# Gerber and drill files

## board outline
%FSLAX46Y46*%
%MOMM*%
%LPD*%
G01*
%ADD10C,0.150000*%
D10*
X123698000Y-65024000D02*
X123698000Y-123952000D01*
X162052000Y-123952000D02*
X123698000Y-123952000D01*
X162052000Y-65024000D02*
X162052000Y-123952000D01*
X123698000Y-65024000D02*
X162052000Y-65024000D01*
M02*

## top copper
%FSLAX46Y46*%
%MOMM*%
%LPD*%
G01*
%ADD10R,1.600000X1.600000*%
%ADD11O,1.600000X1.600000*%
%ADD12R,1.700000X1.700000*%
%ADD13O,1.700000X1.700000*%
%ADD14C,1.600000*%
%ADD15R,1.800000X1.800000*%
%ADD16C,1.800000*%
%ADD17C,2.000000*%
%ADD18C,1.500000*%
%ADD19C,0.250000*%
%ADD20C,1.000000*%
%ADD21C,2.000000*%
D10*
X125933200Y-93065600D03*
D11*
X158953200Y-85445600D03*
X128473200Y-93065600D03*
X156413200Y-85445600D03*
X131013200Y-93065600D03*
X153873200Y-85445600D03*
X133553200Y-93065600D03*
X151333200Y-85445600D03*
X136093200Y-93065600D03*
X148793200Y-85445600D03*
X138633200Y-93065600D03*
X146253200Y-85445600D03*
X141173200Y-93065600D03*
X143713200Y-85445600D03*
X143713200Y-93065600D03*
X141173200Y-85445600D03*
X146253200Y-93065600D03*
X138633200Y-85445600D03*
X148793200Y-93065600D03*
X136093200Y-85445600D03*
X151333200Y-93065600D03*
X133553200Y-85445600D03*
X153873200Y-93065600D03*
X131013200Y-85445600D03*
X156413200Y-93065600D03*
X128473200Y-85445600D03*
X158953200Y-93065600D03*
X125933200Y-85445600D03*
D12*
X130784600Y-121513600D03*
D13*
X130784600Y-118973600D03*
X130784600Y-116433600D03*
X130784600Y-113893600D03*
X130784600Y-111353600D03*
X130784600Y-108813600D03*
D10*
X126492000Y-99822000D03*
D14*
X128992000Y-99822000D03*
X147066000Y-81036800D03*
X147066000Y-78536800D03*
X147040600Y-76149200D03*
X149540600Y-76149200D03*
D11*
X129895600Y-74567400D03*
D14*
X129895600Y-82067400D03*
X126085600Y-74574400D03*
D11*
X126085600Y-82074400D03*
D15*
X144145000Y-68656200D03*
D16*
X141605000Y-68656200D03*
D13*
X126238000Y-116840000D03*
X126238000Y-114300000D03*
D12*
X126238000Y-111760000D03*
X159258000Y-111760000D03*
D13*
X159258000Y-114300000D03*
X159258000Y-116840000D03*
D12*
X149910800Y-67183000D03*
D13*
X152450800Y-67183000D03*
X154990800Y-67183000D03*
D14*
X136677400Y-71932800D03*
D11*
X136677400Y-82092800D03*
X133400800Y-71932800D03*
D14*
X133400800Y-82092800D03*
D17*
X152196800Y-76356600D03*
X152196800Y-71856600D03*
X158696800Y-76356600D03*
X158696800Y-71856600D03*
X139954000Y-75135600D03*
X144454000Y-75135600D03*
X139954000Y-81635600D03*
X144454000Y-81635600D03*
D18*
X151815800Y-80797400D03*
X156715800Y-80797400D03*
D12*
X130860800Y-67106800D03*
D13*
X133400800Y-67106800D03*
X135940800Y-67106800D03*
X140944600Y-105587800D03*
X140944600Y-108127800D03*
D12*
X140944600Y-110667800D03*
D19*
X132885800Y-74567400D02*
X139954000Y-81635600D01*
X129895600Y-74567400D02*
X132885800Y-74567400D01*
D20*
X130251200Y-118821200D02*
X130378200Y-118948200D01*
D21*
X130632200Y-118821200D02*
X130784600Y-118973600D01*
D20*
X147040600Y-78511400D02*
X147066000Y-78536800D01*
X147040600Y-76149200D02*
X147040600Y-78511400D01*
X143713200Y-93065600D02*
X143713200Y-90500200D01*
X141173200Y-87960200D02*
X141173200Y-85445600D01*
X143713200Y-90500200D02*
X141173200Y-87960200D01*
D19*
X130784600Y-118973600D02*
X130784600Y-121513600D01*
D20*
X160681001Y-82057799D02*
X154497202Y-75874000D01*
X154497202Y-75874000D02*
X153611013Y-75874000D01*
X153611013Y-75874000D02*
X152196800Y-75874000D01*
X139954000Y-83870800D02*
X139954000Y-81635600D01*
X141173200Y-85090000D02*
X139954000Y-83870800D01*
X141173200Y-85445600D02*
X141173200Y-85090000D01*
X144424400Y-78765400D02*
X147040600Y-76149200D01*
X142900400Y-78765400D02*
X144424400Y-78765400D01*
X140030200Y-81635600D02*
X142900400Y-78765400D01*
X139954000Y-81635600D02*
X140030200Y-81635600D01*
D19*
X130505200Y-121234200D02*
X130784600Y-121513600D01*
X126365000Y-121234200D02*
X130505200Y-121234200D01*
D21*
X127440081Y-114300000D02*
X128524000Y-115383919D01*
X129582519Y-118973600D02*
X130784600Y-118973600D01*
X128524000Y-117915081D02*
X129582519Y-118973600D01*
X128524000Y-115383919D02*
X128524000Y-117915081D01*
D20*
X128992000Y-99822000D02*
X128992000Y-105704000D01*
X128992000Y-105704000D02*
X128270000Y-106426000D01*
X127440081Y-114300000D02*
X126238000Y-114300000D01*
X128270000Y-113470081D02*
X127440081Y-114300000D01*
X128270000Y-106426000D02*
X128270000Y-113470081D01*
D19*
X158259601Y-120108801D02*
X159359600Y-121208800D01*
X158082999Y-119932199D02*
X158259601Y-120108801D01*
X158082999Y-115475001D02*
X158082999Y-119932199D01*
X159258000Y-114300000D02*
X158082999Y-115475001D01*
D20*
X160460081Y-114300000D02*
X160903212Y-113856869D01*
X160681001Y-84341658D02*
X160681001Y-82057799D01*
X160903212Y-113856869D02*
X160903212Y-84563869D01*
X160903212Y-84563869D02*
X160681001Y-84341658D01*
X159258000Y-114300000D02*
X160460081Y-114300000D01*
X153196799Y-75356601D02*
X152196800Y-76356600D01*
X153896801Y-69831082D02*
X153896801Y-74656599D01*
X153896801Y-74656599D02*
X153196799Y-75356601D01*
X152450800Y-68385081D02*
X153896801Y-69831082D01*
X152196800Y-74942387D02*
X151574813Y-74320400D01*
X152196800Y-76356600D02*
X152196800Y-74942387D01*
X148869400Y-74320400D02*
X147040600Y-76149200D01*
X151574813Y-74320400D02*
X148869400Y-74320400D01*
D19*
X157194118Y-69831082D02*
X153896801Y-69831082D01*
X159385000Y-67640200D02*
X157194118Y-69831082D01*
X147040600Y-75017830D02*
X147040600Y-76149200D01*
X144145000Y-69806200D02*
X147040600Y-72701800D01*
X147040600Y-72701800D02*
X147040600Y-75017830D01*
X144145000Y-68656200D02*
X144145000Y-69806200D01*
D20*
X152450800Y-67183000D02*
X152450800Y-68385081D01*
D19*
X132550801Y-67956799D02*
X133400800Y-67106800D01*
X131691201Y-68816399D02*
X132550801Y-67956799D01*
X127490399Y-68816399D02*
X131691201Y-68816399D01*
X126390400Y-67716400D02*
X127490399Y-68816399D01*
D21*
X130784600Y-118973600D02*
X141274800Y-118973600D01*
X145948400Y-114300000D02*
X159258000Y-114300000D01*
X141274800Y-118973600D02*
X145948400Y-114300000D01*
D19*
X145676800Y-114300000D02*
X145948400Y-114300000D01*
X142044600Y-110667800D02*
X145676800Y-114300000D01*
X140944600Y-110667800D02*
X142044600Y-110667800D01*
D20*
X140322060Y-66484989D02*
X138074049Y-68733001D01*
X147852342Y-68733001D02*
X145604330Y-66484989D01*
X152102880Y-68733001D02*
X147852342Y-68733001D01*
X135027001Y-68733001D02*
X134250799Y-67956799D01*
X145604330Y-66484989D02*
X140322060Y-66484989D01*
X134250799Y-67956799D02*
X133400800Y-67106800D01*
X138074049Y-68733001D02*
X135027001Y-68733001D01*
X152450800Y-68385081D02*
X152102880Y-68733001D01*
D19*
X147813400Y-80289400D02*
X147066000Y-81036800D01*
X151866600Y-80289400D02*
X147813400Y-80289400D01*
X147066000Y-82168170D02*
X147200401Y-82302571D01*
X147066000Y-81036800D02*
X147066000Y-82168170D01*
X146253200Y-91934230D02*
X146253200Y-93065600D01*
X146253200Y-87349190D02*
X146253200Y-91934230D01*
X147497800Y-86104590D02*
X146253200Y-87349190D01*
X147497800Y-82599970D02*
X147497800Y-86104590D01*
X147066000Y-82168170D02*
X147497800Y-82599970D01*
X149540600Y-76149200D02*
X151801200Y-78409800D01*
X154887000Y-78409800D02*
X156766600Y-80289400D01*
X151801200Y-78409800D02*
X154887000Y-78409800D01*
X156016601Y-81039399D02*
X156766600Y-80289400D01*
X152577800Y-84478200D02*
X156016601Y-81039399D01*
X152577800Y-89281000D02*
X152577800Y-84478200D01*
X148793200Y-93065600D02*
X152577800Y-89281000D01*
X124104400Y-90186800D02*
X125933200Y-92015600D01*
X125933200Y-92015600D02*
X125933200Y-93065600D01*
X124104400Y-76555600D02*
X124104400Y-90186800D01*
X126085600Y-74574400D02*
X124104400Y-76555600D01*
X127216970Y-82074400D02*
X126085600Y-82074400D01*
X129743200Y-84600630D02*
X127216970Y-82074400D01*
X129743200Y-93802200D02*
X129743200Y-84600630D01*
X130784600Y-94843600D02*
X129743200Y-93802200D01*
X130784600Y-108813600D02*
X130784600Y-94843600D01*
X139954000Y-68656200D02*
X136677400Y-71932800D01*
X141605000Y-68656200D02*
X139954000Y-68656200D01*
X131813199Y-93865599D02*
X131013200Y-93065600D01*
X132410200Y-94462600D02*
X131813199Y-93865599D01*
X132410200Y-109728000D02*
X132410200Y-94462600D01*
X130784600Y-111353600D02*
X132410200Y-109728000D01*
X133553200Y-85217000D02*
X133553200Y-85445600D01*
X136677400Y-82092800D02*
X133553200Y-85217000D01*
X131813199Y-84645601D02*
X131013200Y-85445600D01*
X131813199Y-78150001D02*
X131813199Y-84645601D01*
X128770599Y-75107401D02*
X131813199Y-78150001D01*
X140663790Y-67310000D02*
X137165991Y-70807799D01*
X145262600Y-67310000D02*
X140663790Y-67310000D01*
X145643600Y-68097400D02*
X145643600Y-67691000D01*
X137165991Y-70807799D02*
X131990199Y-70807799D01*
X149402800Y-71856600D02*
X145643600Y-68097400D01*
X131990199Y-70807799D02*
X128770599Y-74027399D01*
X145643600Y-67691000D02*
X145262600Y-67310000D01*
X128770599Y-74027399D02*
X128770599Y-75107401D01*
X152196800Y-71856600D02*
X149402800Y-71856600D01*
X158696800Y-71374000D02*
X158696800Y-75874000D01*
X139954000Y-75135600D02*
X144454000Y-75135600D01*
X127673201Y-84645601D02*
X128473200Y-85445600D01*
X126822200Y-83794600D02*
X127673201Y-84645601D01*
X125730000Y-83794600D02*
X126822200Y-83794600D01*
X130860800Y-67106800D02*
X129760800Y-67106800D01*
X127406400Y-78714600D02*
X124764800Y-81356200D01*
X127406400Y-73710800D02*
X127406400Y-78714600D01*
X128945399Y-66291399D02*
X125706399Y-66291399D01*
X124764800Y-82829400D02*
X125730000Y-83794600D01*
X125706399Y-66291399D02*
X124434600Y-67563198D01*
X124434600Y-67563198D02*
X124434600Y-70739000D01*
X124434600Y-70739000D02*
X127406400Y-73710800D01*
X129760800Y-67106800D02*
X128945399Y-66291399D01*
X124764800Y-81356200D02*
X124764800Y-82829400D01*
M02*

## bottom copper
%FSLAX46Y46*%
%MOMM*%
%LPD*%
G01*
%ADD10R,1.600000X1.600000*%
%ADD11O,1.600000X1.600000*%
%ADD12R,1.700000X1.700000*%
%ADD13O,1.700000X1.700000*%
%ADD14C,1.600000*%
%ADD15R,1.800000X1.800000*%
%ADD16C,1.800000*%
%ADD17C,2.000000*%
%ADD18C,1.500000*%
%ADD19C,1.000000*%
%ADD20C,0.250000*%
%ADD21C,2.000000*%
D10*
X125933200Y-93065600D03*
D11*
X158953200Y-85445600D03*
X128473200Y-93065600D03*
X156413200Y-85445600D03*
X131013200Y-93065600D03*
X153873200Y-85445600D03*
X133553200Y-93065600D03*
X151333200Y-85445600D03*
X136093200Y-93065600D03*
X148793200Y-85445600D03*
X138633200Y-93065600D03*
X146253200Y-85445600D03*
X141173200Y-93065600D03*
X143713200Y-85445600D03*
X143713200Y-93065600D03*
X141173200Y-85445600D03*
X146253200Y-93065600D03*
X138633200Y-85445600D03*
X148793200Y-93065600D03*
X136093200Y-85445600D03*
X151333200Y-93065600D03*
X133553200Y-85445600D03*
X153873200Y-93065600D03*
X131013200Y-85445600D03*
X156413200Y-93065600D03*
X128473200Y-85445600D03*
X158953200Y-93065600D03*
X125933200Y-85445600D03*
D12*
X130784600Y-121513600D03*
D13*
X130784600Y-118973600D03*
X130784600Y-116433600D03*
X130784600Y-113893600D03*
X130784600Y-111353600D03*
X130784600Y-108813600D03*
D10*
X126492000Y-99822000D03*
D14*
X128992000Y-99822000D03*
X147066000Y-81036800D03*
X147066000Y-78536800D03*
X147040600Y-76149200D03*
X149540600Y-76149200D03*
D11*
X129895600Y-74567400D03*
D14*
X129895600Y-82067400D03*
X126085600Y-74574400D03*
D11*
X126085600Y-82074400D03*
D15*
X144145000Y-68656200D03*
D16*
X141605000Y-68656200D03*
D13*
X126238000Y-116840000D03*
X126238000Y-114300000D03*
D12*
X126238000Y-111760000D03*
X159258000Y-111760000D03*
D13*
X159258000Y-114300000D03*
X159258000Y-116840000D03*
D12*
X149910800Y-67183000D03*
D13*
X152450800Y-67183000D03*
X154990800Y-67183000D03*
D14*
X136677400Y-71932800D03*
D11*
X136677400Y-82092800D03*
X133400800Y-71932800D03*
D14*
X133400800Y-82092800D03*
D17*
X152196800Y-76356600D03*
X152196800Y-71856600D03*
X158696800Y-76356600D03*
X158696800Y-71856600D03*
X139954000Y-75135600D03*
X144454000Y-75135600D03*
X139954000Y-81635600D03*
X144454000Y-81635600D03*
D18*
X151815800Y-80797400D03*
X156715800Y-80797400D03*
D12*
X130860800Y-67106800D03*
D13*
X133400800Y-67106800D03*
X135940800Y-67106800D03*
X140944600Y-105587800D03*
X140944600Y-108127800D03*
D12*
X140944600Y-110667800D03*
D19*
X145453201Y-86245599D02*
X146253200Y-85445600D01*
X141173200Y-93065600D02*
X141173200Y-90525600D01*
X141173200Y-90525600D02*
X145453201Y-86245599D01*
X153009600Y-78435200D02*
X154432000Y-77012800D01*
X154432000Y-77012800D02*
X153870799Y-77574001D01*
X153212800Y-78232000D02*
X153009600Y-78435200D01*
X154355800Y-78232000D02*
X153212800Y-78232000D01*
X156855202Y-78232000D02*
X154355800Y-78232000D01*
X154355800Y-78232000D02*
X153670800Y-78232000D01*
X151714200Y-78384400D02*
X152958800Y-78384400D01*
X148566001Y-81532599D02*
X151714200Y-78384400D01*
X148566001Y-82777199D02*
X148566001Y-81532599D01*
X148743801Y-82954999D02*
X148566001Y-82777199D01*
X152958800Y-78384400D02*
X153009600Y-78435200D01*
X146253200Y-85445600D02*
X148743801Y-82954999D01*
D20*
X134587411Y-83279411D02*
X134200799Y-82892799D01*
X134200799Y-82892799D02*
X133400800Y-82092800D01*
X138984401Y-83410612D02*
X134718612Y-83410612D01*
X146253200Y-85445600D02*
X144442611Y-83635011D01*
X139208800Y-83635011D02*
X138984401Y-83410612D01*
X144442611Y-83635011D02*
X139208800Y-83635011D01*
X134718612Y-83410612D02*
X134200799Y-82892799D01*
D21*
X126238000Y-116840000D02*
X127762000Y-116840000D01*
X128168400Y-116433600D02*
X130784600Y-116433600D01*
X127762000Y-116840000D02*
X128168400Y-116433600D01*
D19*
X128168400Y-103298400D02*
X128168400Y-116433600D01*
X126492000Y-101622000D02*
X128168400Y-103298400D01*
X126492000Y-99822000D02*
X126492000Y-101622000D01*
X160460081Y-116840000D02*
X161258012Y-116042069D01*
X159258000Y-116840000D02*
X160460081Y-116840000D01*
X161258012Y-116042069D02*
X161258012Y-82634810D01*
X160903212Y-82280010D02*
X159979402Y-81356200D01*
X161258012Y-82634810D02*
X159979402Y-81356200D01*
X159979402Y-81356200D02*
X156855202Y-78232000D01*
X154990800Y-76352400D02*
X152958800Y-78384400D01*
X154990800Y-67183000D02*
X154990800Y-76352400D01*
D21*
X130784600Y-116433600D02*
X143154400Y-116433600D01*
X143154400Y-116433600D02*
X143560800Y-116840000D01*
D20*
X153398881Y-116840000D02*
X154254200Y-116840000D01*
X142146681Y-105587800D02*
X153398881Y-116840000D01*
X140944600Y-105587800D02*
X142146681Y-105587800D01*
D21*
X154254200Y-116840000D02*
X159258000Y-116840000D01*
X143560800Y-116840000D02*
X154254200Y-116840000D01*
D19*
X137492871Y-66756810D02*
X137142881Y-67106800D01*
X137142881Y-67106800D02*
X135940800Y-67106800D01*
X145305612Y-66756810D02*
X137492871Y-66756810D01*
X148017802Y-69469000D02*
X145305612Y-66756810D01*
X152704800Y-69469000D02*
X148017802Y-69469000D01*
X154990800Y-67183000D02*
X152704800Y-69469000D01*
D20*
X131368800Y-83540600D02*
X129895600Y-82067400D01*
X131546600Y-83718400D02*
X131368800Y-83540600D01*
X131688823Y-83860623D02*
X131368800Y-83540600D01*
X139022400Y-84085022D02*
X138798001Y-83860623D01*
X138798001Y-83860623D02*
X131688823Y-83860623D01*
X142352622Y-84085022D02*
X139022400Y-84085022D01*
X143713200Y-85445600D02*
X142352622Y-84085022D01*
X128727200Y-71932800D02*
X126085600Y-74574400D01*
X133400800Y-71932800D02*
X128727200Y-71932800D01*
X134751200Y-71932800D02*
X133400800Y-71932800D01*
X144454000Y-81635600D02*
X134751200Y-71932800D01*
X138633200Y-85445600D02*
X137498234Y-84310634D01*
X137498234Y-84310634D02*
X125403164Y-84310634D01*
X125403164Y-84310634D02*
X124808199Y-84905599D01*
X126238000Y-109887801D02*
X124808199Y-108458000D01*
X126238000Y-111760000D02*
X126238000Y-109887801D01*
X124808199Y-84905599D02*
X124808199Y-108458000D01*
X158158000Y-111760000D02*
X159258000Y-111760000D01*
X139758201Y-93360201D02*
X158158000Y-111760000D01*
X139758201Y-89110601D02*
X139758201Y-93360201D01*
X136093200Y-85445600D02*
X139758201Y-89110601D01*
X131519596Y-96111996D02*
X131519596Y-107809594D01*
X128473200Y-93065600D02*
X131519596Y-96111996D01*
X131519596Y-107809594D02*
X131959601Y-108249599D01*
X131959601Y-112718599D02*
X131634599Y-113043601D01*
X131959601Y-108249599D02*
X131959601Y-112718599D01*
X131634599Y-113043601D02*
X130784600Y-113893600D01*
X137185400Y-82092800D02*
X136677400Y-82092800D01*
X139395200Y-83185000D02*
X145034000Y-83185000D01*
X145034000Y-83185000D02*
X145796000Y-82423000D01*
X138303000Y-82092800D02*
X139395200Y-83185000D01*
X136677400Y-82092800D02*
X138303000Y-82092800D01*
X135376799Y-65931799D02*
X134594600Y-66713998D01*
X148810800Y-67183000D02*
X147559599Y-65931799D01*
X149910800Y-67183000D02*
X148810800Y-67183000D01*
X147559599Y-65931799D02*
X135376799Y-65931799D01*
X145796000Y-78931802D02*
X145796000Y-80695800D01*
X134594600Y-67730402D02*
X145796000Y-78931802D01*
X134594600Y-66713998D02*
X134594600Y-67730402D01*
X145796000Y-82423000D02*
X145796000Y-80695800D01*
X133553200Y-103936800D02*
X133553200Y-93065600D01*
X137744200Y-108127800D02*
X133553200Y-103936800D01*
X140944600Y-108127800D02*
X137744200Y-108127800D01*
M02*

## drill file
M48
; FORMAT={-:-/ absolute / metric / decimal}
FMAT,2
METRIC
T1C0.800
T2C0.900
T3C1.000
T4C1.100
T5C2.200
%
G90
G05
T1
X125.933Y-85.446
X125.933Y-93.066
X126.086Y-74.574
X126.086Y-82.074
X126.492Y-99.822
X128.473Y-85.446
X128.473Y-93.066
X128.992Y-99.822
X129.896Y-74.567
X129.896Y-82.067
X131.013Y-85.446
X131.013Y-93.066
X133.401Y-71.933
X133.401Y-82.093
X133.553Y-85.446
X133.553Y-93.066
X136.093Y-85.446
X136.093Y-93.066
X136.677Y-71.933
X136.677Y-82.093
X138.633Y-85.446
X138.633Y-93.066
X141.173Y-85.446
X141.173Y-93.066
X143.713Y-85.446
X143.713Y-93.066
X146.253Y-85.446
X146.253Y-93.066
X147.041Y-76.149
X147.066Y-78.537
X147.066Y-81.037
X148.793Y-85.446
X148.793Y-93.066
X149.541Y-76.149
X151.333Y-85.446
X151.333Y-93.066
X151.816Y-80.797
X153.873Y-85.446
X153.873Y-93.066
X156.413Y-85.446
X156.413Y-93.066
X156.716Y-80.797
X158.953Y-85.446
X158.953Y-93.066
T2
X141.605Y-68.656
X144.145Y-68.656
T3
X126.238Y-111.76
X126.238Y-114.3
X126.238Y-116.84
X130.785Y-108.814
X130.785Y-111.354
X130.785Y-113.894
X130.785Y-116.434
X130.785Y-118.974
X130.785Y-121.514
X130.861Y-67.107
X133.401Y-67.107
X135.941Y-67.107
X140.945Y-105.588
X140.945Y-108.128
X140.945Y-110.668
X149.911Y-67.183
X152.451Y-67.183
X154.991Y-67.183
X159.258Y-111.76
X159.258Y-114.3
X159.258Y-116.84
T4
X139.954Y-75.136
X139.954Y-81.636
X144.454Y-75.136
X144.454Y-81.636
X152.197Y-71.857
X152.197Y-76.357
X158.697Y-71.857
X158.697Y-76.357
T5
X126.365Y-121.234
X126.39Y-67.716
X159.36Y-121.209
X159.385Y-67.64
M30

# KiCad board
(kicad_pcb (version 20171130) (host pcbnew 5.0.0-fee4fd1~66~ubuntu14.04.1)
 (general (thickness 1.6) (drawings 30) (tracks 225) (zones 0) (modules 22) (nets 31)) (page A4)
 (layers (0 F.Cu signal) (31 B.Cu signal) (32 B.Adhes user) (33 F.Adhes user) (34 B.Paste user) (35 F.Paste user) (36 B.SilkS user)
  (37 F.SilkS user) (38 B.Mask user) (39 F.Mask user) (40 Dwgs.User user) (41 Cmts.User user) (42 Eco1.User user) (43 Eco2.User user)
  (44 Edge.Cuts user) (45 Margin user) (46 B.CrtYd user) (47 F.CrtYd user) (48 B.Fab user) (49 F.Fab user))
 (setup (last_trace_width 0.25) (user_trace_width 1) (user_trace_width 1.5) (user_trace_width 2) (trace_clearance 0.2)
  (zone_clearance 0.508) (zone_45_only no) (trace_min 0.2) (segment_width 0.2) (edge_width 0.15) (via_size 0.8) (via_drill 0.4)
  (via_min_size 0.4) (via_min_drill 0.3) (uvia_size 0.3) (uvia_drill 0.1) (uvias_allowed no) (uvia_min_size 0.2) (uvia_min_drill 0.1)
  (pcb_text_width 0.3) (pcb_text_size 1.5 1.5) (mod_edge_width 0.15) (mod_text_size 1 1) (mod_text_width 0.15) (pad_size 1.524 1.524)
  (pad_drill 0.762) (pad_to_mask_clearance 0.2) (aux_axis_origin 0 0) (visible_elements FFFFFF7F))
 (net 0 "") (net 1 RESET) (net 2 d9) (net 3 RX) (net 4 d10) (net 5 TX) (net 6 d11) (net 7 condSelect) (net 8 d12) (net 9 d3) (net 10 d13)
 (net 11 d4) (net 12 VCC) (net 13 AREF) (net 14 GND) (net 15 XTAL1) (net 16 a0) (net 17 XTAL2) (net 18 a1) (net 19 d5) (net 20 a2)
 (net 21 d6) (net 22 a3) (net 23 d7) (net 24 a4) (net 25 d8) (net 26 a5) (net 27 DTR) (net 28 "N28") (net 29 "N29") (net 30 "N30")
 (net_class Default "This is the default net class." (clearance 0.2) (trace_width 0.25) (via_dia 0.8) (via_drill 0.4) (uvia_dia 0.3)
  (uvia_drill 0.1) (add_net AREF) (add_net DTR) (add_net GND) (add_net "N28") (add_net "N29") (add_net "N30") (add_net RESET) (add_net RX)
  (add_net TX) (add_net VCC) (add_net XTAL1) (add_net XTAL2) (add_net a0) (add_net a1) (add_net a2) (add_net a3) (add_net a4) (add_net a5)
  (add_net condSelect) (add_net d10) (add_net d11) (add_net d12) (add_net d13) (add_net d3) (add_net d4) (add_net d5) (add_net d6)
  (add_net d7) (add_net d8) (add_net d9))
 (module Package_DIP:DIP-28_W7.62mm (layer F.Cu) (at 125.9332 93.0656 90)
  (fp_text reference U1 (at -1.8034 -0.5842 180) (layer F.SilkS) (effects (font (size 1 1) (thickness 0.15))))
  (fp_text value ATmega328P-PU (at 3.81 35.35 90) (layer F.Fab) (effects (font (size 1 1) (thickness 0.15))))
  (pad 1 thru_hole rect (at 0 0 90) (size 1.6 1.6) (drill 0.8) (layers *.Cu *.Mask) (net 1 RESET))
  (pad 15 thru_hole oval (at 7.62 33.02 90) (size 1.6 1.6) (drill 0.8) (layers *.Cu *.Mask) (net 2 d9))
  (pad 2 thru_hole oval (at 0 2.54 90) (size 1.6 1.6) (drill 0.8) (layers *.Cu *.Mask) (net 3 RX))
  (pad 16 thru_hole oval (at 7.62 30.48 90) (size 1.6 1.6) (drill 0.8) (layers *.Cu *.Mask) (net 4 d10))
  (pad 3 thru_hole oval (at 0 5.08 90) (size 1.6 1.6) (drill 0.8) (layers *.Cu *.Mask) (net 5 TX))
  (pad 17 thru_hole oval (at 7.62 27.94 90) (size 1.6 1.6) (drill 0.8) (layers *.Cu *.Mask) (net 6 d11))
  (pad 4 thru_hole oval (at 0 7.62 90) (size 1.6 1.6) (drill 0.8) (layers *.Cu *.Mask) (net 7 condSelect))
  (pad 18 thru_hole oval (at 7.62 25.4 90) (size 1.6 1.6) (drill 0.8) (layers *.Cu *.Mask) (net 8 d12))
  (pad 5 thru_hole oval (at 0 10.16 90) (size 1.6 1.6) (drill 0.8) (layers *.Cu *.Mask) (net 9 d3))
  (pad 19 thru_hole oval (at 7.62 22.86 90) (size 1.6 1.6) (drill 0.8) (layers *.Cu *.Mask) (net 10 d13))
  (pad 6 thru_hole oval (at 0 12.7 90) (size 1.6 1.6) (drill 0.8) (layers *.Cu *.Mask) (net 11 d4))
  (pad 20 thru_hole oval (at 7.62 20.32 90) (size 1.6 1.6) (drill 0.8) (layers *.Cu *.Mask) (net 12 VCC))
  (pad 7 thru_hole oval (at 0 15.24 90) (size 1.6 1.6) (drill 0.8) (layers *.Cu *.Mask) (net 12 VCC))
  (pad 21 thru_hole oval (at 7.62 17.78 90) (size 1.6 1.6) (drill 0.8) (layers *.Cu *.Mask) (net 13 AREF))
  (pad 8 thru_hole oval (at 0 17.78 90) (size 1.6 1.6) (drill 0.8) (layers *.Cu *.Mask) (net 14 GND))
  (pad 22 thru_hole oval (at 7.62 15.24 90) (size 1.6 1.6) (drill 0.8) (layers *.Cu *.Mask) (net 14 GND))
  (pad 9 thru_hole oval (at 0 20.32 90) (size 1.6 1.6) (drill 0.8) (layers *.Cu *.Mask) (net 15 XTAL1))
  (pad 23 thru_hole oval (at 7.62 12.7 90) (size 1.6 1.6) (drill 0.8) (layers *.Cu *.Mask) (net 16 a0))
  (pad 10 thru_hole oval (at 0 22.86 90) (size 1.6 1.6) (drill 0.8) (layers *.Cu *.Mask) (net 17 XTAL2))
  (pad 24 thru_hole oval (at 7.62 10.16 90) (size 1.6 1.6) (drill 0.8) (layers *.Cu *.Mask) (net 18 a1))
  (pad 11 thru_hole oval (at 0 25.4 90) (size 1.6 1.6) (drill 0.8) (layers *.Cu *.Mask) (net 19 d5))
  (pad 25 thru_hole oval (at 7.62 7.62 90) (size 1.6 1.6) (drill 0.8) (layers *.Cu *.Mask) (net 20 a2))
  (pad 12 thru_hole oval (at 0 27.94 90) (size 1.6 1.6) (drill 0.8) (layers *.Cu *.Mask) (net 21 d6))
  (pad 26 thru_hole oval (at 7.62 5.08 90) (size 1.6 1.6) (drill 0.8) (layers *.Cu *.Mask) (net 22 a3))
  (pad 13 thru_hole oval (at 0 30.48 90) (size 1.6 1.6) (drill 0.8) (layers *.Cu *.Mask) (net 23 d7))
  (pad 27 thru_hole oval (at 7.62 2.54 90) (size 1.6 1.6) (drill 0.8) (layers *.Cu *.Mask) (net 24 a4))
  (pad 14 thru_hole oval (at 0 33.02 90) (size 1.6 1.6) (drill 0.8) (layers *.Cu *.Mask) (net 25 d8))
  (pad 28 thru_hole oval (at 7.62 0 90) (size 1.6 1.6) (drill 0.8) (layers *.Cu *.Mask) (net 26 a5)))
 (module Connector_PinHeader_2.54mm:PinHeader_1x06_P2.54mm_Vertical (layer F.Cu) (at 130.7846 121.5136 180)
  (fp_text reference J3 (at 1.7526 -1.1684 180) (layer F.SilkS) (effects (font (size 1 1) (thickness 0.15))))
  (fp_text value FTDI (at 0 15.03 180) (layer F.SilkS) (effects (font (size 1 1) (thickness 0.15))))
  (pad 1 thru_hole rect (at 0 0 180) (size 1.7 1.7) (drill 1) (layers *.Cu *.Mask) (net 14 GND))
  (pad 2 thru_hole oval (at 0 2.54 180) (size 1.7 1.7) (drill 1) (layers *.Cu *.Mask) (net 14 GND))
  (pad 3 thru_hole oval (at 0 5.08 180) (size 1.7 1.7) (drill 1) (layers *.Cu *.Mask) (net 12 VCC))
  (pad 4 thru_hole oval (at 0 7.62 180) (size 1.7 1.7) (drill 1) (layers *.Cu *.Mask) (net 3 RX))
  (pad 5 thru_hole oval (at 0 10.16 180) (size 1.7 1.7) (drill 1) (layers *.Cu *.Mask) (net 5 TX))
  (pad 6 thru_hole oval (at 0 12.7 180) (size 1.7 1.7) (drill 1) (layers *.Cu *.Mask) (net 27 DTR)))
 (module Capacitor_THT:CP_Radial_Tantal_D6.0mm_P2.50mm (layer F.Cu) (at 126.492 99.822)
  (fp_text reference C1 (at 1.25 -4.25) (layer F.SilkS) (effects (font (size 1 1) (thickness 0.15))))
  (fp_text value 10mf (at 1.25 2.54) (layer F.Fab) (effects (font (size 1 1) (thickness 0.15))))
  (pad 1 thru_hole rect (at 0 0) (size 1.6 1.6) (drill 0.8) (layers *.Cu *.Mask) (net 12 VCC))
  (pad 2 thru_hole circle (at 2.5 0) (size 1.6 1.6) (drill 0.8) (layers *.Cu *.Mask) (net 14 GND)))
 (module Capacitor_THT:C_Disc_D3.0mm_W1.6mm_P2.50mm (layer F.Cu) (at 147.066 78.5368 270)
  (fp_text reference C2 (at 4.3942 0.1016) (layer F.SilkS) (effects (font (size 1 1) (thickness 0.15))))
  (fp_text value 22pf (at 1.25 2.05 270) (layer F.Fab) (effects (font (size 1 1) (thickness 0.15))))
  (pad 2 thru_hole circle (at 2.5 0 270) (size 1.6 1.6) (drill 0.8) (layers *.Cu *.Mask) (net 15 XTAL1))
  (pad 1 thru_hole circle (at 0 0 270) (size 1.6 1.6) (drill 0.8) (layers *.Cu *.Mask) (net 14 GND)))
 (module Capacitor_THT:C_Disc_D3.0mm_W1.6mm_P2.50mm (layer F.Cu) (at 147.0406 76.1492)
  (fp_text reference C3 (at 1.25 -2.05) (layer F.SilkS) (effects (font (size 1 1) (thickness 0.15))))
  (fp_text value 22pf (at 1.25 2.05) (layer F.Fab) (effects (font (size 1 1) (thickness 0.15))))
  (pad 1 thru_hole circle (at 0 0) (size 1.6 1.6) (drill 0.8) (layers *.Cu *.Mask) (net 14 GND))
  (pad 2 thru_hole circle (at 2.5 0) (size 1.6 1.6) (drill 0.8) (layers *.Cu *.Mask) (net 17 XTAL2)))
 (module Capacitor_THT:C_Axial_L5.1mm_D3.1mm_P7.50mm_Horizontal (layer F.Cu) (at 129.8956 82.0674 90)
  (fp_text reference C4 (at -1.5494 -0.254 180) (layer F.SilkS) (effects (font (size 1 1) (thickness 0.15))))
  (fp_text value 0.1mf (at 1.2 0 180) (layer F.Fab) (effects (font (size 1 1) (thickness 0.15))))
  (pad 2 thru_hole oval (at 7.5 0 90) (size 1.6 1.6) (drill 0.8) (layers *.Cu *.Mask) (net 14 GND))
  (pad 1 thru_hole circle (at 0 0 90) (size 1.6 1.6) (drill 0.8) (layers *.Cu *.Mask) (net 13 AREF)))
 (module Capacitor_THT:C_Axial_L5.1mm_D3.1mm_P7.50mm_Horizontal (layer F.Cu) (at 126.0856 74.5744 270)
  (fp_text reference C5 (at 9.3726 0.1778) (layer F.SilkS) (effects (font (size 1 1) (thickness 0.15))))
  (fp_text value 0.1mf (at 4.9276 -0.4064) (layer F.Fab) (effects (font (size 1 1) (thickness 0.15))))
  (pad 1 thru_hole circle (at 0 0 270) (size 1.6 1.6) (drill 0.8) (layers *.Cu *.Mask) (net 1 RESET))
  (pad 2 thru_hole oval (at 7.5 0 270) (size 1.6 1.6) (drill 0.8) (layers *.Cu *.Mask) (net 27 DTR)))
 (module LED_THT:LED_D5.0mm (layer F.Cu) (at 144.145 68.6562 180)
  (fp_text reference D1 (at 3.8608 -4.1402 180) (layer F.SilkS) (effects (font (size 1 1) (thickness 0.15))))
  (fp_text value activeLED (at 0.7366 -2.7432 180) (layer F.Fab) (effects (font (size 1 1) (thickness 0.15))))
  (pad 1 thru_hole rect (at 0 0 180) (size 1.8 1.8) (drill 0.9) (layers *.Cu *.Mask) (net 14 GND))
  (pad 2 thru_hole circle (at 2.54 0 180) (size 1.8 1.8) (drill 0.9) (layers *.Cu *.Mask) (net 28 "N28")))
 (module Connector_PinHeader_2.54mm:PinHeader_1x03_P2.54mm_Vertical (layer F.Cu) (at 126.238 111.76)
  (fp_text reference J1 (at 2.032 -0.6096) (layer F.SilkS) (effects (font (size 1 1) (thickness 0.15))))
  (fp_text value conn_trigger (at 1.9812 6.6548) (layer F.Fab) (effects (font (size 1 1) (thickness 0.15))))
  (pad 3 thru_hole oval (at 0 5.08) (size 1.7 1.7) (drill 1) (layers *.Cu *.Mask) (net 12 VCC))
  (pad 2 thru_hole oval (at 0 2.54) (size 1.7 1.7) (drill 1) (layers *.Cu *.Mask) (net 14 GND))
  (pad 1 thru_hole rect (at 0 0) (size 1.7 1.7) (drill 1) (layers *.Cu *.Mask) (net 16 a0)))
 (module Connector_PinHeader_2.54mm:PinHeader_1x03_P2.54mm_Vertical (layer F.Cu) (at 159.258 111.76)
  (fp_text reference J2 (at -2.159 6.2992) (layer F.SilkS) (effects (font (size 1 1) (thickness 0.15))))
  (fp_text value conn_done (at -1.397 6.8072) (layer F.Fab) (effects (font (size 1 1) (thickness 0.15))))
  (pad 1 thru_hole rect (at 0 0) (size 1.7 1.7) (drill 1) (layers *.Cu *.Mask) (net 18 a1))
  (pad 2 thru_hole oval (at 0 2.54) (size 1.7 1.7) (drill 1) (layers *.Cu *.Mask) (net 14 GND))
  (pad 3 thru_hole oval (at 0 5.08) (size 1.7 1.7) (drill 1) (layers *.Cu *.Mask) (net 12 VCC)))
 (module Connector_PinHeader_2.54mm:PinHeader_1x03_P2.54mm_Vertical (layer F.Cu) (at 149.9108 67.183 90)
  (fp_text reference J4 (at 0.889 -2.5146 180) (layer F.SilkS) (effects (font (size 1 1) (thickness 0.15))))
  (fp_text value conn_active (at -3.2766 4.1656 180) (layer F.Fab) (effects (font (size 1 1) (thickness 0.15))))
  (pad 1 thru_hole rect (at 0 0 90) (size 1.7 1.7) (drill 1) (layers *.Cu *.Mask) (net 20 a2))
  (pad 2 thru_hole oval (at 0 2.54 90) (size 1.7 1.7) (drill 1) (layers *.Cu *.Mask) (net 14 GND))
  (pad 3 thru_hole oval (at 0 5.08 90) (size 1.7 1.7) (drill 1) (layers *.Cu *.Mask) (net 12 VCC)))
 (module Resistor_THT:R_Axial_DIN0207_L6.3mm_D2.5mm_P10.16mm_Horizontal (layer F.Cu) (at 136.6774 71.9328 270)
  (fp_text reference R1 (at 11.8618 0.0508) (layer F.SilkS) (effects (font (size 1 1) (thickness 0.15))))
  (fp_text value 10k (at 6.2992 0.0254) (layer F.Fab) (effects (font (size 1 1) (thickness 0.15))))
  (pad 1 thru_hole circle (at 0 0 270) (size 1.6 1.6) (drill 0.8) (layers *.Cu *.Mask) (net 28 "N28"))
  (pad 2 thru_hole oval (at 10.16 0 270) (size 1.6 1.6) (drill 0.8) (layers *.Cu *.Mask) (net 20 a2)))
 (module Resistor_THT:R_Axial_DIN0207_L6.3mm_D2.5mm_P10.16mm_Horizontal (layer F.Cu) (at 133.4008 82.0928 90)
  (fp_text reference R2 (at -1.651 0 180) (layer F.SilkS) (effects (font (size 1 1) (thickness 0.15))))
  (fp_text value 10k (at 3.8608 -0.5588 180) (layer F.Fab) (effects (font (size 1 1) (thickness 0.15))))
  (pad 2 thru_hole oval (at 10.16 0 90) (size 1.6 1.6) (drill 0.8) (layers *.Cu *.Mask) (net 1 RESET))
  (pad 1 thru_hole circle (at 0 0 90) (size 1.6 1.6) (drill 0.8) (layers *.Cu *.Mask) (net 12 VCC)))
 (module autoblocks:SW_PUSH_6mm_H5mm (layer F.Cu) (at 152.1968 71.8566)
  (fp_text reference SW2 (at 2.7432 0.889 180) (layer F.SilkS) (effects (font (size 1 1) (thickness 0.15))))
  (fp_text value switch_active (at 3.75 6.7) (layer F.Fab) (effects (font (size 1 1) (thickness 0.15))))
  (pad 2 thru_hole circle (at 0 4.5 90) (size 2 2) (drill 1.1) (layers *.Cu *.Mask) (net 14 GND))
  (pad 1 thru_hole circle (at 0 0 90) (size 2 2) (drill 1.1) (layers *.Cu *.Mask) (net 22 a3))
  (pad 4 thru_hole circle (at 6.5 4.5 90) (size 2 2) (drill 1.1) (layers *.Cu *.Mask) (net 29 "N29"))
  (pad 3 thru_hole circle (at 6.5 0 90) (size 2 2) (drill 1.1) (layers *.Cu *.Mask) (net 29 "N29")))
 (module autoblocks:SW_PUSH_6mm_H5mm (layer F.Cu) (at 139.954 81.6356 90)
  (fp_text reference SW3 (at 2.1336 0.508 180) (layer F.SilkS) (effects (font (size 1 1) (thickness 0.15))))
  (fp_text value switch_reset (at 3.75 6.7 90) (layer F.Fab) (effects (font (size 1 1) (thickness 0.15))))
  (pad 3 thru_hole circle (at 6.5 0 180) (size 2 2) (drill 1.1) (layers *.Cu *.Mask) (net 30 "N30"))
  (pad 4 thru_hole circle (at 6.5 4.5 180) (size 2 2) (drill 1.1) (layers *.Cu *.Mask) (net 30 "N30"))
  (pad 1 thru_hole circle (at 0 0 180) (size 2 2) (drill 1.1) (layers *.Cu *.Mask) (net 14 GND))
  (pad 2 thru_hole circle (at 0 4.5 180) (size 2 2) (drill 1.1) (layers *.Cu *.Mask) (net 1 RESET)))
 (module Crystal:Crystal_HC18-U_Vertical (layer F.Cu) (at 151.8158 80.7974)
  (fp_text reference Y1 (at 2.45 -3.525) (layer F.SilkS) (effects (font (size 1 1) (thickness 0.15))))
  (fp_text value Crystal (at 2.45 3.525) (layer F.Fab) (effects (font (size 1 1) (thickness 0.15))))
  (pad 1 thru_hole circle (at 0 0) (size 1.5 1.5) (drill 0.8) (layers *.Cu *.Mask) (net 15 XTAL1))
  (pad 2 thru_hole circle (at 4.9 0) (size 1.5 1.5) (drill 0.8) (layers *.Cu *.Mask) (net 17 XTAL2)))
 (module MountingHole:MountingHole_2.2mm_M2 (layer F.Cu) (at 126.365 121.2342)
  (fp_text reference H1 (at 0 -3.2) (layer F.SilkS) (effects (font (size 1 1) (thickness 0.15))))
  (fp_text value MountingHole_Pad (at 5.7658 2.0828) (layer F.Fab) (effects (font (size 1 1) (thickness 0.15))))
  (pad 1 np_thru_hole circle (at 0 0) (size 2.2 2.2) (drill 2.2) (layers *.Cu *.Mask) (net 14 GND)))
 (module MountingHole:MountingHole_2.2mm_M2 (layer F.Cu) (at 159.3596 121.2088)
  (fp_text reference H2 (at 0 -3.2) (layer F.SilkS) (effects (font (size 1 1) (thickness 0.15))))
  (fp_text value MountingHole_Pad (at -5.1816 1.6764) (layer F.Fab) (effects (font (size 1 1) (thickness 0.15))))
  (pad 1 np_thru_hole circle (at 0 0) (size 2.2 2.2) (drill 2.2) (layers *.Cu *.Mask) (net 14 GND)))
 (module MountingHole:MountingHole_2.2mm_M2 (layer F.Cu) (at 159.385 67.6402)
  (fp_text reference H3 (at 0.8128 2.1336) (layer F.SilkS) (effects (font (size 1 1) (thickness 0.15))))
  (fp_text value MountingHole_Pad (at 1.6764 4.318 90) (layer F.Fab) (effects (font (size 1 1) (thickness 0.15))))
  (pad 1 np_thru_hole circle (at 0 0) (size 2.2 2.2) (drill 2.2) (layers *.Cu *.Mask) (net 14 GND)))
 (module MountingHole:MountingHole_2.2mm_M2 (layer F.Cu) (at 126.3904 67.7164)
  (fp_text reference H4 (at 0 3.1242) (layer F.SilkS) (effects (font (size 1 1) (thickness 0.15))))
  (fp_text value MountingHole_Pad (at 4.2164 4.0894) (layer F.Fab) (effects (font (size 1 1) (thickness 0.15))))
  (pad 1 np_thru_hole circle (at 0 0) (size 2.2 2.2) (drill 2.2) (layers *.Cu *.Mask) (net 14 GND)))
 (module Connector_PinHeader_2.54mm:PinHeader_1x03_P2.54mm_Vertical (layer F.Cu) (at 130.8608 67.1068 90)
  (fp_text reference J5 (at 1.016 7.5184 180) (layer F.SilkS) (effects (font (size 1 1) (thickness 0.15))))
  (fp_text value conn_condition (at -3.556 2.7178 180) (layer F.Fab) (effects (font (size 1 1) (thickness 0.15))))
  (pad 1 thru_hole rect (at 0 0 90) (size 1.7 1.7) (drill 1) (layers *.Cu *.Mask) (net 24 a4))
  (pad 2 thru_hole oval (at 0 2.54 90) (size 1.7 1.7) (drill 1) (layers *.Cu *.Mask) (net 14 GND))
  (pad 3 thru_hole oval (at 0 5.08 90) (size 1.7 1.7) (drill 1) (layers *.Cu *.Mask) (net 12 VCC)))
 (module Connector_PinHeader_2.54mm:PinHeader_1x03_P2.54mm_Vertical (layer F.Cu) (at 140.9446 110.6678 180)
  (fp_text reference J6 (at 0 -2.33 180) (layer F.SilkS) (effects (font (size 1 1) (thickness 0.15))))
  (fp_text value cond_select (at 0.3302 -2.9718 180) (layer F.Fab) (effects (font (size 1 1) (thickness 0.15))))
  (pad 3 thru_hole oval (at 0 5.08 180) (size 1.7 1.7) (drill 1) (layers *.Cu *.Mask) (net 12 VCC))
  (pad 2 thru_hole oval (at 0 2.54 180) (size 1.7 1.7) (drill 1) (layers *.Cu *.Mask) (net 7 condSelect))
  (pad 1 thru_hole rect (at 0 0 180) (size 1.7 1.7) (drill 1) (layers *.Cu *.Mask) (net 14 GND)))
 (gr_line (start 123.698 65.024) (end 123.698 123.952) (layer Edge.Cuts) (width 0.15))
 (gr_line (start 162.052 123.952) (end 123.698 123.952) (layer Edge.Cuts) (width 0.15))
 (gr_line (start 162.052 65.024) (end 162.052 123.952) (layer Edge.Cuts) (width 0.15))
 (gr_line (start 123.698 65.024) (end 162.052 65.024) (layer Edge.Cuts) (width 0.15))
 (segment (start 132.8858 74.5674) (end 139.954 81.6356) (width 0.25) (layer F.Cu) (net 14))
 (segment (start 129.8956 74.5674) (end 132.8858 74.5674) (width 0.25) (layer F.Cu) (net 14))
 (segment (start 130.2512 118.8212) (end 130.3782 118.9482) (width 1) (layer F.Cu) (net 14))
 (segment (start 130.6322 118.8212) (end 130.7846 118.9736) (width 2) (layer F.Cu) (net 14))
 (segment (start 147.0406 78.5114) (end 147.066 78.5368) (width 1) (layer F.Cu) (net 14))
 (segment (start 147.0406 76.1492) (end 147.0406 78.5114) (width 1) (layer F.Cu) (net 14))
 (segment (start 143.7132 93.0656) (end 143.7132 90.5002) (width 1) (layer F.Cu) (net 14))
 (segment (start 141.1732 87.9602) (end 141.1732 85.4456) (width 1) (layer F.Cu) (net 14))
 (segment (start 143.7132 90.5002) (end 141.1732 87.9602) (width 1) (layer F.Cu) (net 14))
 (segment (start 130.7846 118.9736) (end 130.7846 121.5136) (width 0.25) (layer F.Cu) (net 14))
 (segment (start 160.681001 82.057799) (end 154.497202 75.874) (width 1) (layer F.Cu) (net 14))
 (segment (start 154.497202 75.874) (end 153.611013 75.874) (width 1) (layer F.Cu) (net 14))
 (segment (start 153.611013 75.874) (end 152.1968 75.874) (width 1) (layer F.Cu) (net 14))
 (segment (start 139.954 83.8708) (end 139.954 81.6356) (width 1) (layer F.Cu) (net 14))
 (segment (start 141.1732 85.09) (end 139.954 83.8708) (width 1) (layer F.Cu) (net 14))
 (segment (start 141.1732 85.4456) (end 141.1732 85.09) (width 1) (layer F.Cu) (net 14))
 (segment (start 144.4244 78.7654) (end 147.0406 76.1492) (width 1) (layer F.Cu) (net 14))
 (segment (start 142.9004 78.7654) (end 144.4244 78.7654) (width 1) (layer F.Cu) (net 14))
 (segment (start 140.0302 81.6356) (end 142.9004 78.7654) (width 1) (layer F.Cu) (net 14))
 (segment (start 139.954 81.6356) (end 140.0302 81.6356) (width 1) (layer F.Cu) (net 14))
 (segment (start 130.5052 121.2342) (end 130.7846 121.5136) (width 0.25) (layer F.Cu) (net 14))
 (segment (start 126.365 121.2342) (end 130.5052 121.2342) (width 0.25) (layer F.Cu) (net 14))
 (segment (start 127.440081 114.3) (end 128.524 115.383919) (width 2) (layer F.Cu) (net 14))
 (segment (start 129.582519 118.9736) (end 130.7846 118.9736) (width 2) (layer F.Cu) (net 14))
 (segment (start 128.524 117.915081) (end 129.582519 118.9736) (width 2) (layer F.Cu) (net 14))
 (segment (start 128.524 115.383919) (end 128.524 117.915081) (width 2) (layer F.Cu) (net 14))
 (segment (start 128.992 99.822) (end 128.992 105.704) (width 1) (layer F.Cu) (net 14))
 (segment (start 128.992 105.704) (end 128.27 106.426) (width 1) (layer F.Cu) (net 14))
 (segment (start 127.440081 114.3) (end 126.238 114.3) (width 1) (layer F.Cu) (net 14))
 (segment (start 128.27 113.470081) (end 127.440081 114.3) (width 1) (layer F.Cu) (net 14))
 (segment (start 128.27 106.426) (end 128.27 113.470081) (width 1) (layer F.Cu) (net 14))
 (segment (start 158.259601 120.108801) (end 159.3596 121.2088) (width 0.25) (layer F.Cu) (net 14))
 (segment (start 158.082999 119.932199) (end 158.259601 120.108801) (width 0.25) (layer F.Cu) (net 14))
 (segment (start 158.082999 115.475001) (end 158.082999 119.932199) (width 0.25) (layer F.Cu) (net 14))
 (segment (start 159.258 114.3) (end 158.082999 115.475001) (width 0.25) (layer F.Cu) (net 14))
 (segment (start 160.460081 114.3) (end 160.903212 113.856869) (width 1) (layer F.Cu) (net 14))
 (segment (start 160.681001 84.341658) (end 160.681001 82.057799) (width 1) (layer F.Cu) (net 14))
 (segment (start 160.903212 113.856869) (end 160.903212 84.563869) (width 1) (layer F.Cu) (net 14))
 (segment (start 160.903212 84.563869) (end 160.681001 84.341658) (width 1) (layer F.Cu) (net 14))
 (segment (start 159.258 114.3) (end 160.460081 114.3) (width 1) (layer F.Cu) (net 14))
 (segment (start 153.196799 75.356601) (end 152.1968 76.3566) (width 1) (layer F.Cu) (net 14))
 (segment (start 153.896801 69.831082) (end 153.896801 74.656599) (width 1) (layer F.Cu) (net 14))
 (segment (start 153.896801 74.656599) (end 153.196799 75.356601) (width 1) (layer F.Cu) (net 14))
 (segment (start 152.4508 68.385081) (end 153.896801 69.831082) (width 1) (layer F.Cu) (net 14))
 (segment (start 152.1968 74.942387) (end 151.574813 74.3204) (width 1) (layer F.Cu) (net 14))
 (segment (start 152.1968 76.3566) (end 152.1968 74.942387) (width 1) (layer F.Cu) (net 14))
 (segment (start 148.8694 74.3204) (end 147.0406 76.1492) (width 1) (layer F.Cu) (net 14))
 (segment (start 151.574813 74.3204) (end 148.8694 74.3204) (width 1) (layer F.Cu) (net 14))
 (segment (start 157.194118 69.831082) (end 153.896801 69.831082) (width 0.25) (layer F.Cu) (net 14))
 (segment (start 159.385 67.6402) (end 157.194118 69.831082) (width 0.25) (layer F.Cu) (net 14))
 (segment (start 147.0406 75.01783) (end 147.0406 76.1492) (width 0.25) (layer F.Cu) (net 14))
 (segment (start 144.145 69.8062) (end 147.0406 72.7018) (width 0.25) (layer F.Cu) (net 14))
 (segment (start 147.0406 72.7018) (end 147.0406 75.01783) (width 0.25) (layer F.Cu) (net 14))
 (segment (start 144.145 68.6562) (end 144.145 69.8062) (width 0.25) (layer F.Cu) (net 14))
 (segment (start 152.4508 67.183) (end 152.4508 68.385081) (width 1) (layer F.Cu) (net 14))
 (segment (start 132.550801 67.956799) (end 133.4008 67.1068) (width 0.25) (layer F.Cu) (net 14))
 (segment (start 131.691201 68.816399) (end 132.550801 67.956799) (width 0.25) (layer F.Cu) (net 14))
 (segment (start 127.490399 68.816399) (end 131.691201 68.816399) (width 0.25) (layer F.Cu) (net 14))
 (segment (start 126.3904 67.7164) (end 127.490399 68.816399) (width 0.25) (layer F.Cu) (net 14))
 (segment (start 130.7846 118.9736) (end 141.2748 118.9736) (width 2) (layer F.Cu) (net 14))
 (segment (start 145.9484 114.3) (end 159.258 114.3) (width 2) (layer F.Cu) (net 14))
 (segment (start 141.2748 118.9736) (end 145.9484 114.3) (width 2) (layer F.Cu) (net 14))
 (segment (start 145.6768 114.3) (end 145.9484 114.3) (width 0.25) (layer F.Cu) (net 14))
 (segment (start 142.0446 110.6678) (end 145.6768 114.3) (width 0.25) (layer F.Cu) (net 14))
 (segment (start 140.9446 110.6678) (end 142.0446 110.6678) (width 0.25) (layer F.Cu) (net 14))
 (segment (start 140.32206 66.484989) (end 138.074049 68.733001) (width 1) (layer F.Cu) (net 14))
 (segment (start 147.852342 68.733001) (end 145.60433 66.484989) (width 1) (layer F.Cu) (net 14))
 (segment (start 152.10288 68.733001) (end 147.852342 68.733001) (width 1) (layer F.Cu) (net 14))
 (segment (start 135.027001 68.733001) (end 134.250799 67.956799) (width 1) (layer F.Cu) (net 14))
 (segment (start 145.60433 66.484989) (end 140.32206 66.484989) (width 1) (layer F.Cu) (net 14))
 (segment (start 134.250799 67.956799) (end 133.4008 67.1068) (width 1) (layer F.Cu) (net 14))
 (segment (start 138.074049 68.733001) (end 135.027001 68.733001) (width 1) (layer F.Cu) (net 14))
 (segment (start 152.4508 68.385081) (end 152.10288 68.733001) (width 1) (layer F.Cu) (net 14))
 (segment (start 145.453201 86.245599) (end 146.2532 85.4456) (width 1) (layer B.Cu) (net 12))
 (segment (start 141.1732 93.0656) (end 141.1732 90.5256) (width 1) (layer B.Cu) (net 12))
 (segment (start 141.1732 90.5256) (end 145.453201 86.245599) (width 1) (layer B.Cu) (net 12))
 (segment (start 153.0096 78.4352) (end 154.432 77.0128) (width 1) (layer B.Cu) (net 12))
 (segment (start 154.432 77.0128) (end 153.870799 77.574001) (width 1) (layer B.Cu) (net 12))
 (segment (start 153.2128 78.232) (end 153.0096 78.4352) (width 1) (layer B.Cu) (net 12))
 (segment (start 154.3558 78.232) (end 153.2128 78.232) (width 1) (layer B.Cu) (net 12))
 (segment (start 156.855202 78.232) (end 154.3558 78.232) (width 1) (layer B.Cu) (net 12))
 (segment (start 154.3558 78.232) (end 153.6708 78.232) (width 1) (layer B.Cu) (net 12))
 (segment (start 151.7142 78.3844) (end 152.9588 78.3844) (width 1) (layer B.Cu) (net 12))
 (segment (start 148.566001 81.532599) (end 151.7142 78.3844) (width 1) (layer B.Cu) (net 12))
 (segment (start 148.566001 82.777199) (end 148.566001 81.532599) (width 1) (layer B.Cu) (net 12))
 (segment (start 148.743801 82.954999) (end 148.566001 82.777199) (width 1) (layer B.Cu) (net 12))
 (segment (start 152.9588 78.3844) (end 153.0096 78.4352) (width 1) (layer B.Cu) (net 12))
 (segment (start 146.2532 85.4456) (end 148.743801 82.954999) (width 1) (layer B.Cu) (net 12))
 (segment (start 134.587411 83.279411) (end 134.200799 82.892799) (width 0.25) (layer B.Cu) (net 12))
 (segment (start 134.200799 82.892799) (end 133.4008 82.0928) (width 0.25) (layer B.Cu) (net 12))
 (segment (start 138.984401 83.410612) (end 134.718612 83.410612) (width 0.25) (layer B.Cu) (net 12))
 (segment (start 146.2532 85.4456) (end 144.442611 83.635011) (width 0.25) (layer B.Cu) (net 12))
 (segment (start 139.2088 83.635011) (end 138.984401 83.410612) (width 0.25) (layer B.Cu) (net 12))
 (segment (start 144.442611 83.635011) (end 139.2088 83.635011) (width 0.25) (layer B.Cu) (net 12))
 (segment (start 134.718612 83.410612) (end 134.200799 82.892799) (width 0.25) (layer B.Cu) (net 12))
 (segment (start 126.238 116.84) (end 127.762 116.84) (width 2) (layer B.Cu) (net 12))
 (segment (start 128.1684 116.4336) (end 130.7846 116.4336) (width 2) (layer B.Cu) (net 12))
 (segment (start 127.762 116.84) (end 128.1684 116.4336) (width 2) (layer B.Cu) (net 12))
 (segment (start 128.1684 103.2984) (end 128.1684 116.4336) (width 1) (layer B.Cu) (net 12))
 (segment (start 126.492 101.622) (end 128.1684 103.2984) (width 1) (layer B.Cu) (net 12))
 (segment (start 126.492 99.822) (end 126.492 101.622) (width 1) (layer B.Cu) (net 12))
 (segment (start 160.460081 116.84) (end 161.258012 116.042069) (width 1) (layer B.Cu) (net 12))
 (segment (start 159.258 116.84) (end 160.460081 116.84) (width 1) (layer B.Cu) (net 12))
 (segment (start 161.258012 116.042069) (end 161.258012 82.63481) (width 1) (layer B.Cu) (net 12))
 (segment (start 160.903212 82.28001) (end 159.979402 81.3562) (width 1) (layer B.Cu) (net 12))
 (segment (start 161.258012 82.63481) (end 159.979402 81.3562) (width 1) (layer B.Cu) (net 12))
 (segment (start 159.979402 81.3562) (end 156.855202 78.232) (width 1) (layer B.Cu) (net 12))
 (segment (start 154.9908 76.3524) (end 152.9588 78.3844) (width 1) (layer B.Cu) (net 12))
 (segment (start 154.9908 67.183) (end 154.9908 76.3524) (width 1) (layer B.Cu) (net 12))
 (segment (start 130.7846 116.4336) (end 143.1544 116.4336) (width 2) (layer B.Cu) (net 12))
 (segment (start 143.1544 116.4336) (end 143.5608 116.84) (width 2) (layer B.Cu) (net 12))
 (segment (start 153.398881 116.84) (end 154.2542 116.84) (width 0.25) (layer B.Cu) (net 12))
 (segment (start 142.146681 105.5878) (end 153.398881 116.84) (width 0.25) (layer B.Cu) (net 12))
 (segment (start 140.9446 105.5878) (end 142.146681 105.5878) (width 0.25) (layer B.Cu) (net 12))
 (segment (start 154.2542 116.84) (end 159.258 116.84) (width 2) (layer B.Cu) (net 12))
 (segment (start 143.5608 116.84) (end 154.2542 116.84) (width 2) (layer B.Cu) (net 12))
 (segment (start 137.492871 66.75681) (end 137.142881 67.1068) (width 1) (layer B.Cu) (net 12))
 (segment (start 137.142881 67.1068) (end 135.9408 67.1068) (width 1) (layer B.Cu) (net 12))
 (segment (start 145.305612 66.75681) (end 137.492871 66.75681) (width 1) (layer B.Cu) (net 12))
 (segment (start 148.017802 69.469) (end 145.305612 66.75681) (width 1) (layer B.Cu) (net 12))
 (segment (start 152.7048 69.469) (end 148.017802 69.469) (width 1) (layer B.Cu) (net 12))
 (segment (start 154.9908 67.183) (end 152.7048 69.469) (width 1) (layer B.Cu) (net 12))
 (segment (start 147.8134 80.2894) (end 147.066 81.0368) (width 0.25) (layer F.Cu) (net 15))
 (segment (start 151.8666 80.2894) (end 147.8134 80.2894) (width 0.25) (layer F.Cu) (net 15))
 (segment (start 147.066 82.16817) (end 147.200401 82.302571) (width 0.25) (layer F.Cu) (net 15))
 (segment (start 147.066 81.0368) (end 147.066 82.16817) (width 0.25) (layer F.Cu) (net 15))
 (segment (start 146.2532 91.93423) (end 146.2532 93.0656) (width 0.25) (layer F.Cu) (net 15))
 (segment (start 146.2532 87.34919) (end 146.2532 91.93423) (width 0.25) (layer F.Cu) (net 15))
 (segment (start 147.4978 86.10459) (end 146.2532 87.34919) (width 0.25) (layer F.Cu) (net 15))
 (segment (start 147.4978 82.59997) (end 147.4978 86.10459) (width 0.25) (layer F.Cu) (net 15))
 (segment (start 147.066 82.16817) (end 147.4978 82.59997) (width 0.25) (layer F.Cu) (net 15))
 (segment (start 149.5406 76.1492) (end 151.8012 78.4098) (width 0.25) (layer F.Cu) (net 17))
 (segment (start 154.887 78.4098) (end 156.7666 80.2894) (width 0.25) (layer F.Cu) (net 17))
 (segment (start 151.8012 78.4098) (end 154.887 78.4098) (width 0.25) (layer F.Cu) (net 17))
 (segment (start 156.016601 81.039399) (end 156.7666 80.2894) (width 0.25) (layer F.Cu) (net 17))
 (segment (start 152.5778 84.4782) (end 156.016601 81.039399) (width 0.25) (layer F.Cu) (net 17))
 (segment (start 152.5778 89.281) (end 152.5778 84.4782) (width 0.25) (layer F.Cu) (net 17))
 (segment (start 148.7932 93.0656) (end 152.5778 89.281) (width 0.25) (layer F.Cu) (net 17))
 (segment (start 131.3688 83.5406) (end 129.8956 82.0674) (width 0.25) (layer B.Cu) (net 13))
 (segment (start 131.5466 83.7184) (end 131.3688 83.5406) (width 0.25) (layer B.Cu) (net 13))
 (segment (start 131.688823 83.860623) (end 131.3688 83.5406) (width 0.25) (layer B.Cu) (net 13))
 (segment (start 139.0224 84.085022) (end 138.798001 83.860623) (width 0.25) (layer B.Cu) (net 13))
 (segment (start 138.798001 83.860623) (end 131.688823 83.860623) (width 0.25) (layer B.Cu) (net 13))
 (segment (start 142.352622 84.085022) (end 139.0224 84.085022) (width 0.25) (layer B.Cu) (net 13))
 (segment (start 143.7132 85.4456) (end 142.352622 84.085022) (width 0.25) (layer B.Cu) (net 13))
 (segment (start 128.7272 71.9328) (end 126.0856 74.5744) (width 0.25) (layer B.Cu) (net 1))
 (segment (start 133.4008 71.9328) (end 128.7272 71.9328) (width 0.25) (layer B.Cu) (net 1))
 (segment (start 134.7512 71.9328) (end 133.4008 71.9328) (width 0.25) (layer B.Cu) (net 1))
 (segment (start 144.454 81.6356) (end 134.7512 71.9328) (width 0.25) (layer B.Cu) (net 1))
 (segment (start 124.1044 90.1868) (end 125.9332 92.0156) (width 0.25) (layer F.Cu) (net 1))
 (segment (start 125.9332 92.0156) (end 125.9332 93.0656) (width 0.25) (layer F.Cu) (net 1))
 (segment (start 124.1044 76.5556) (end 124.1044 90.1868) (width 0.25) (layer F.Cu) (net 1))
 (segment (start 126.0856 74.5744) (end 124.1044 76.5556) (width 0.25) (layer F.Cu) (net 1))
 (segment (start 127.21697 82.0744) (end 126.0856 82.0744) (width 0.25) (layer F.Cu) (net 27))
 (segment (start 129.7432 84.60063) (end 127.21697 82.0744) (width 0.25) (layer F.Cu) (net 27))
 (segment (start 129.7432 93.8022) (end 129.7432 84.60063) (width 0.25) (layer F.Cu) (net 27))
 (segment (start 130.7846 94.8436) (end 129.7432 93.8022) (width 0.25) (layer F.Cu) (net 27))
 (segment (start 130.7846 108.8136) (end 130.7846 94.8436) (width 0.25) (layer F.Cu) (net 27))
 (segment (start 139.954 68.6562) (end 136.6774 71.9328) (width 0.25) (layer F.Cu) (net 28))
 (segment (start 141.605 68.6562) (end 139.954 68.6562) (width 0.25) (layer F.Cu) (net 28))
 (segment (start 138.6332 85.4456) (end 137.498234 84.310634) (width 0.25) (layer B.Cu) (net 16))
 (segment (start 137.498234 84.310634) (end 125.403164 84.310634) (width 0.25) (layer B.Cu) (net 16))
 (segment (start 125.403164 84.310634) (end 124.808199 84.905599) (width 0.25) (layer B.Cu) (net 16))
 (segment (start 126.238 109.887801) (end 124.808199 108.458) (width 0.25) (layer B.Cu) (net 16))
 (segment (start 126.238 111.76) (end 126.238 109.887801) (width 0.25) (layer B.Cu) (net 16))
 (segment (start 124.808199 84.905599) (end 124.808199 108.458) (width 0.25) (layer B.Cu) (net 16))
 (segment (start 158.158 111.76) (end 159.258 111.76) (width 0.25) (layer B.Cu) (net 18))
 (segment (start 139.758201 93.360201) (end 158.158 111.76) (width 0.25) (layer B.Cu) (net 18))
 (segment (start 139.758201 89.110601) (end 139.758201 93.360201) (width 0.25) (layer B.Cu) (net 18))
 (segment (start 136.0932 85.4456) (end 139.758201 89.110601) (width 0.25) (layer B.Cu) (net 18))
 (segment (start 131.519596 96.111996) (end 131.519596 107.809594) (width 0.25) (layer B.Cu) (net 3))
 (segment (start 128.4732 93.0656) (end 131.519596 96.111996) (width 0.25) (layer B.Cu) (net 3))
 (segment (start 131.519596 107.809594) (end 131.959601 108.249599) (width 0.25) (layer B.Cu) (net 3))
 (segment (start 131.959601 112.718599) (end 131.634599 113.043601) (width 0.25) (layer B.Cu) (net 3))
 (segment (start 131.959601 108.249599) (end 131.959601 112.718599) (width 0.25) (layer B.Cu) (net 3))
 (segment (start 131.634599 113.043601) (end 130.7846 113.8936) (width 0.25) (layer B.Cu) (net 3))
 (segment (start 131.813199 93.865599) (end 131.0132 93.0656) (width 0.25) (layer F.Cu) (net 5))
 (segment (start 132.4102 94.4626) (end 131.813199 93.865599) (width 0.25) (layer F.Cu) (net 5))
 (segment (start 132.4102 109.728) (end 132.4102 94.4626) (width 0.25) (layer F.Cu) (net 5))
 (segment (start 130.7846 111.3536) (end 132.4102 109.728) (width 0.25) (layer F.Cu) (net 5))
 (segment (start 137.1854 82.0928) (end 136.6774 82.0928) (width 0.25) (layer B.Cu) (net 20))
 (segment (start 133.5532 85.217) (end 133.5532 85.4456) (width 0.25) (layer F.Cu) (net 20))
 (segment (start 136.6774 82.0928) (end 133.5532 85.217) (width 0.25) (layer F.Cu) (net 20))
 (segment (start 139.3952 83.185) (end 145.034 83.185) (width 0.25) (layer B.Cu) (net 20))
 (segment (start 145.034 83.185) (end 145.796 82.423) (width 0.25) (layer B.Cu) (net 20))
 (segment (start 138.303 82.0928) (end 139.3952 83.185) (width 0.25) (layer B.Cu) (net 20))
 (segment (start 136.6774 82.0928) (end 138.303 82.0928) (width 0.25) (layer B.Cu) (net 20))
 (segment (start 135.376799 65.931799) (end 134.5946 66.713998) (width 0.25) (layer B.Cu) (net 20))
 (segment (start 148.8108 67.183) (end 147.559599 65.931799) (width 0.25) (layer B.Cu) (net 20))
 (segment (start 149.9108 67.183) (end 148.8108 67.183) (width 0.25) (layer B.Cu) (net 20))
 (segment (start 147.559599 65.931799) (end 135.376799 65.931799) (width 0.25) (layer B.Cu) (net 20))
 (segment (start 145.796 78.931802) (end 145.796 80.6958) (width 0.25) (layer B.Cu) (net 20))
 (segment (start 134.5946 67.730402) (end 145.796 78.931802) (width 0.25) (layer B.Cu) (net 20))
 (segment (start 134.5946 66.713998) (end 134.5946 67.730402) (width 0.25) (layer B.Cu) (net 20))
 (segment (start 145.796 82.423) (end 145.796 80.6958) (width 0.25) (layer B.Cu) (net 20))
 (segment (start 131.813199 84.645601) (end 131.0132 85.4456) (width 0.25) (layer F.Cu) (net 22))
 (segment (start 131.813199 78.150001) (end 131.813199 84.645601) (width 0.25) (layer F.Cu) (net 22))
 (segment (start 128.770599 75.107401) (end 131.813199 78.150001) (width 0.25) (layer F.Cu) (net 22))
 (segment (start 140.66379 67.31) (end 137.165991 70.807799) (width 0.25) (layer F.Cu) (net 22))
 (segment (start 145.2626 67.31) (end 140.66379 67.31) (width 0.25) (layer F.Cu) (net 22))
 (segment (start 145.6436 68.0974) (end 145.6436 67.691) (width 0.25) (layer F.Cu) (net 22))
 (segment (start 137.165991 70.807799) (end 131.990199 70.807799) (width 0.25) (layer F.Cu) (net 22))
 (segment (start 149.4028 71.8566) (end 145.6436 68.0974) (width 0.25) (layer F.Cu) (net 22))
 (segment (start 131.990199 70.807799) (end 128.770599 74.027399) (width 0.25) (layer F.Cu) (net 22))
 (segment (start 145.6436 67.691) (end 145.2626 67.31) (width 0.25) (layer F.Cu) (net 22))
 (segment (start 128.770599 74.027399) (end 128.770599 75.107401) (width 0.25) (layer F.Cu) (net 22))
 (segment (start 152.1968 71.8566) (end 149.4028 71.8566) (width 0.25) (layer F.Cu) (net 22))
 (segment (start 158.6968 71.374) (end 158.6968 75.874) (width 0.25) (layer F.Cu) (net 29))
 (segment (start 139.954 75.1356) (end 144.454 75.1356) (width 0.25) (layer F.Cu) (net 30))
 (segment (start 127.673201 84.645601) (end 128.4732 85.4456) (width 0.25) (layer F.Cu) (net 24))
 (segment (start 126.8222 83.7946) (end 127.673201 84.645601) (width 0.25) (layer F.Cu) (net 24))
 (segment (start 125.73 83.7946) (end 126.8222 83.7946) (width 0.25) (layer F.Cu) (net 24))
 (segment (start 130.8608 67.1068) (end 129.7608 67.1068) (width 0.25) (layer F.Cu) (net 24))
 (segment (start 127.4064 78.7146) (end 124.7648 81.3562) (width 0.25) (layer F.Cu) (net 24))
 (segment (start 127.4064 73.7108) (end 127.4064 78.7146) (width 0.25) (layer F.Cu) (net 24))
 (segment (start 128.945399 66.291399) (end 125.706399 66.291399) (width 0.25) (layer F.Cu) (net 24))
 (segment (start 124.7648 82.8294) (end 125.73 83.7946) (width 0.25) (layer F.Cu) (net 24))
 (segment (start 125.706399 66.291399) (end 124.4346 67.563198) (width 0.25) (layer F.Cu) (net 24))
 (segment (start 124.4346 67.563198) (end 124.4346 70.739) (width 0.25) (layer F.Cu) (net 24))
 (segment (start 124.4346 70.739) (end 127.4064 73.7108) (width 0.25) (layer F.Cu) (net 24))
 (segment (start 129.7608 67.1068) (end 128.945399 66.291399) (width 0.25) (layer F.Cu) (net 24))
 (segment (start 124.7648 81.3562) (end 124.7648 82.8294) (width 0.25) (layer F.Cu) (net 24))
 (segment (start 133.5532 103.9368) (end 133.5532 93.0656) (width 0.25) (layer B.Cu) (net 7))
 (segment (start 137.7442 108.1278) (end 133.5532 103.9368) (width 0.25) (layer B.Cu) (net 7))
 (segment (start 140.9446 108.1278) (end 137.7442 108.1278) (width 0.25) (layer B.Cu) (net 7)))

